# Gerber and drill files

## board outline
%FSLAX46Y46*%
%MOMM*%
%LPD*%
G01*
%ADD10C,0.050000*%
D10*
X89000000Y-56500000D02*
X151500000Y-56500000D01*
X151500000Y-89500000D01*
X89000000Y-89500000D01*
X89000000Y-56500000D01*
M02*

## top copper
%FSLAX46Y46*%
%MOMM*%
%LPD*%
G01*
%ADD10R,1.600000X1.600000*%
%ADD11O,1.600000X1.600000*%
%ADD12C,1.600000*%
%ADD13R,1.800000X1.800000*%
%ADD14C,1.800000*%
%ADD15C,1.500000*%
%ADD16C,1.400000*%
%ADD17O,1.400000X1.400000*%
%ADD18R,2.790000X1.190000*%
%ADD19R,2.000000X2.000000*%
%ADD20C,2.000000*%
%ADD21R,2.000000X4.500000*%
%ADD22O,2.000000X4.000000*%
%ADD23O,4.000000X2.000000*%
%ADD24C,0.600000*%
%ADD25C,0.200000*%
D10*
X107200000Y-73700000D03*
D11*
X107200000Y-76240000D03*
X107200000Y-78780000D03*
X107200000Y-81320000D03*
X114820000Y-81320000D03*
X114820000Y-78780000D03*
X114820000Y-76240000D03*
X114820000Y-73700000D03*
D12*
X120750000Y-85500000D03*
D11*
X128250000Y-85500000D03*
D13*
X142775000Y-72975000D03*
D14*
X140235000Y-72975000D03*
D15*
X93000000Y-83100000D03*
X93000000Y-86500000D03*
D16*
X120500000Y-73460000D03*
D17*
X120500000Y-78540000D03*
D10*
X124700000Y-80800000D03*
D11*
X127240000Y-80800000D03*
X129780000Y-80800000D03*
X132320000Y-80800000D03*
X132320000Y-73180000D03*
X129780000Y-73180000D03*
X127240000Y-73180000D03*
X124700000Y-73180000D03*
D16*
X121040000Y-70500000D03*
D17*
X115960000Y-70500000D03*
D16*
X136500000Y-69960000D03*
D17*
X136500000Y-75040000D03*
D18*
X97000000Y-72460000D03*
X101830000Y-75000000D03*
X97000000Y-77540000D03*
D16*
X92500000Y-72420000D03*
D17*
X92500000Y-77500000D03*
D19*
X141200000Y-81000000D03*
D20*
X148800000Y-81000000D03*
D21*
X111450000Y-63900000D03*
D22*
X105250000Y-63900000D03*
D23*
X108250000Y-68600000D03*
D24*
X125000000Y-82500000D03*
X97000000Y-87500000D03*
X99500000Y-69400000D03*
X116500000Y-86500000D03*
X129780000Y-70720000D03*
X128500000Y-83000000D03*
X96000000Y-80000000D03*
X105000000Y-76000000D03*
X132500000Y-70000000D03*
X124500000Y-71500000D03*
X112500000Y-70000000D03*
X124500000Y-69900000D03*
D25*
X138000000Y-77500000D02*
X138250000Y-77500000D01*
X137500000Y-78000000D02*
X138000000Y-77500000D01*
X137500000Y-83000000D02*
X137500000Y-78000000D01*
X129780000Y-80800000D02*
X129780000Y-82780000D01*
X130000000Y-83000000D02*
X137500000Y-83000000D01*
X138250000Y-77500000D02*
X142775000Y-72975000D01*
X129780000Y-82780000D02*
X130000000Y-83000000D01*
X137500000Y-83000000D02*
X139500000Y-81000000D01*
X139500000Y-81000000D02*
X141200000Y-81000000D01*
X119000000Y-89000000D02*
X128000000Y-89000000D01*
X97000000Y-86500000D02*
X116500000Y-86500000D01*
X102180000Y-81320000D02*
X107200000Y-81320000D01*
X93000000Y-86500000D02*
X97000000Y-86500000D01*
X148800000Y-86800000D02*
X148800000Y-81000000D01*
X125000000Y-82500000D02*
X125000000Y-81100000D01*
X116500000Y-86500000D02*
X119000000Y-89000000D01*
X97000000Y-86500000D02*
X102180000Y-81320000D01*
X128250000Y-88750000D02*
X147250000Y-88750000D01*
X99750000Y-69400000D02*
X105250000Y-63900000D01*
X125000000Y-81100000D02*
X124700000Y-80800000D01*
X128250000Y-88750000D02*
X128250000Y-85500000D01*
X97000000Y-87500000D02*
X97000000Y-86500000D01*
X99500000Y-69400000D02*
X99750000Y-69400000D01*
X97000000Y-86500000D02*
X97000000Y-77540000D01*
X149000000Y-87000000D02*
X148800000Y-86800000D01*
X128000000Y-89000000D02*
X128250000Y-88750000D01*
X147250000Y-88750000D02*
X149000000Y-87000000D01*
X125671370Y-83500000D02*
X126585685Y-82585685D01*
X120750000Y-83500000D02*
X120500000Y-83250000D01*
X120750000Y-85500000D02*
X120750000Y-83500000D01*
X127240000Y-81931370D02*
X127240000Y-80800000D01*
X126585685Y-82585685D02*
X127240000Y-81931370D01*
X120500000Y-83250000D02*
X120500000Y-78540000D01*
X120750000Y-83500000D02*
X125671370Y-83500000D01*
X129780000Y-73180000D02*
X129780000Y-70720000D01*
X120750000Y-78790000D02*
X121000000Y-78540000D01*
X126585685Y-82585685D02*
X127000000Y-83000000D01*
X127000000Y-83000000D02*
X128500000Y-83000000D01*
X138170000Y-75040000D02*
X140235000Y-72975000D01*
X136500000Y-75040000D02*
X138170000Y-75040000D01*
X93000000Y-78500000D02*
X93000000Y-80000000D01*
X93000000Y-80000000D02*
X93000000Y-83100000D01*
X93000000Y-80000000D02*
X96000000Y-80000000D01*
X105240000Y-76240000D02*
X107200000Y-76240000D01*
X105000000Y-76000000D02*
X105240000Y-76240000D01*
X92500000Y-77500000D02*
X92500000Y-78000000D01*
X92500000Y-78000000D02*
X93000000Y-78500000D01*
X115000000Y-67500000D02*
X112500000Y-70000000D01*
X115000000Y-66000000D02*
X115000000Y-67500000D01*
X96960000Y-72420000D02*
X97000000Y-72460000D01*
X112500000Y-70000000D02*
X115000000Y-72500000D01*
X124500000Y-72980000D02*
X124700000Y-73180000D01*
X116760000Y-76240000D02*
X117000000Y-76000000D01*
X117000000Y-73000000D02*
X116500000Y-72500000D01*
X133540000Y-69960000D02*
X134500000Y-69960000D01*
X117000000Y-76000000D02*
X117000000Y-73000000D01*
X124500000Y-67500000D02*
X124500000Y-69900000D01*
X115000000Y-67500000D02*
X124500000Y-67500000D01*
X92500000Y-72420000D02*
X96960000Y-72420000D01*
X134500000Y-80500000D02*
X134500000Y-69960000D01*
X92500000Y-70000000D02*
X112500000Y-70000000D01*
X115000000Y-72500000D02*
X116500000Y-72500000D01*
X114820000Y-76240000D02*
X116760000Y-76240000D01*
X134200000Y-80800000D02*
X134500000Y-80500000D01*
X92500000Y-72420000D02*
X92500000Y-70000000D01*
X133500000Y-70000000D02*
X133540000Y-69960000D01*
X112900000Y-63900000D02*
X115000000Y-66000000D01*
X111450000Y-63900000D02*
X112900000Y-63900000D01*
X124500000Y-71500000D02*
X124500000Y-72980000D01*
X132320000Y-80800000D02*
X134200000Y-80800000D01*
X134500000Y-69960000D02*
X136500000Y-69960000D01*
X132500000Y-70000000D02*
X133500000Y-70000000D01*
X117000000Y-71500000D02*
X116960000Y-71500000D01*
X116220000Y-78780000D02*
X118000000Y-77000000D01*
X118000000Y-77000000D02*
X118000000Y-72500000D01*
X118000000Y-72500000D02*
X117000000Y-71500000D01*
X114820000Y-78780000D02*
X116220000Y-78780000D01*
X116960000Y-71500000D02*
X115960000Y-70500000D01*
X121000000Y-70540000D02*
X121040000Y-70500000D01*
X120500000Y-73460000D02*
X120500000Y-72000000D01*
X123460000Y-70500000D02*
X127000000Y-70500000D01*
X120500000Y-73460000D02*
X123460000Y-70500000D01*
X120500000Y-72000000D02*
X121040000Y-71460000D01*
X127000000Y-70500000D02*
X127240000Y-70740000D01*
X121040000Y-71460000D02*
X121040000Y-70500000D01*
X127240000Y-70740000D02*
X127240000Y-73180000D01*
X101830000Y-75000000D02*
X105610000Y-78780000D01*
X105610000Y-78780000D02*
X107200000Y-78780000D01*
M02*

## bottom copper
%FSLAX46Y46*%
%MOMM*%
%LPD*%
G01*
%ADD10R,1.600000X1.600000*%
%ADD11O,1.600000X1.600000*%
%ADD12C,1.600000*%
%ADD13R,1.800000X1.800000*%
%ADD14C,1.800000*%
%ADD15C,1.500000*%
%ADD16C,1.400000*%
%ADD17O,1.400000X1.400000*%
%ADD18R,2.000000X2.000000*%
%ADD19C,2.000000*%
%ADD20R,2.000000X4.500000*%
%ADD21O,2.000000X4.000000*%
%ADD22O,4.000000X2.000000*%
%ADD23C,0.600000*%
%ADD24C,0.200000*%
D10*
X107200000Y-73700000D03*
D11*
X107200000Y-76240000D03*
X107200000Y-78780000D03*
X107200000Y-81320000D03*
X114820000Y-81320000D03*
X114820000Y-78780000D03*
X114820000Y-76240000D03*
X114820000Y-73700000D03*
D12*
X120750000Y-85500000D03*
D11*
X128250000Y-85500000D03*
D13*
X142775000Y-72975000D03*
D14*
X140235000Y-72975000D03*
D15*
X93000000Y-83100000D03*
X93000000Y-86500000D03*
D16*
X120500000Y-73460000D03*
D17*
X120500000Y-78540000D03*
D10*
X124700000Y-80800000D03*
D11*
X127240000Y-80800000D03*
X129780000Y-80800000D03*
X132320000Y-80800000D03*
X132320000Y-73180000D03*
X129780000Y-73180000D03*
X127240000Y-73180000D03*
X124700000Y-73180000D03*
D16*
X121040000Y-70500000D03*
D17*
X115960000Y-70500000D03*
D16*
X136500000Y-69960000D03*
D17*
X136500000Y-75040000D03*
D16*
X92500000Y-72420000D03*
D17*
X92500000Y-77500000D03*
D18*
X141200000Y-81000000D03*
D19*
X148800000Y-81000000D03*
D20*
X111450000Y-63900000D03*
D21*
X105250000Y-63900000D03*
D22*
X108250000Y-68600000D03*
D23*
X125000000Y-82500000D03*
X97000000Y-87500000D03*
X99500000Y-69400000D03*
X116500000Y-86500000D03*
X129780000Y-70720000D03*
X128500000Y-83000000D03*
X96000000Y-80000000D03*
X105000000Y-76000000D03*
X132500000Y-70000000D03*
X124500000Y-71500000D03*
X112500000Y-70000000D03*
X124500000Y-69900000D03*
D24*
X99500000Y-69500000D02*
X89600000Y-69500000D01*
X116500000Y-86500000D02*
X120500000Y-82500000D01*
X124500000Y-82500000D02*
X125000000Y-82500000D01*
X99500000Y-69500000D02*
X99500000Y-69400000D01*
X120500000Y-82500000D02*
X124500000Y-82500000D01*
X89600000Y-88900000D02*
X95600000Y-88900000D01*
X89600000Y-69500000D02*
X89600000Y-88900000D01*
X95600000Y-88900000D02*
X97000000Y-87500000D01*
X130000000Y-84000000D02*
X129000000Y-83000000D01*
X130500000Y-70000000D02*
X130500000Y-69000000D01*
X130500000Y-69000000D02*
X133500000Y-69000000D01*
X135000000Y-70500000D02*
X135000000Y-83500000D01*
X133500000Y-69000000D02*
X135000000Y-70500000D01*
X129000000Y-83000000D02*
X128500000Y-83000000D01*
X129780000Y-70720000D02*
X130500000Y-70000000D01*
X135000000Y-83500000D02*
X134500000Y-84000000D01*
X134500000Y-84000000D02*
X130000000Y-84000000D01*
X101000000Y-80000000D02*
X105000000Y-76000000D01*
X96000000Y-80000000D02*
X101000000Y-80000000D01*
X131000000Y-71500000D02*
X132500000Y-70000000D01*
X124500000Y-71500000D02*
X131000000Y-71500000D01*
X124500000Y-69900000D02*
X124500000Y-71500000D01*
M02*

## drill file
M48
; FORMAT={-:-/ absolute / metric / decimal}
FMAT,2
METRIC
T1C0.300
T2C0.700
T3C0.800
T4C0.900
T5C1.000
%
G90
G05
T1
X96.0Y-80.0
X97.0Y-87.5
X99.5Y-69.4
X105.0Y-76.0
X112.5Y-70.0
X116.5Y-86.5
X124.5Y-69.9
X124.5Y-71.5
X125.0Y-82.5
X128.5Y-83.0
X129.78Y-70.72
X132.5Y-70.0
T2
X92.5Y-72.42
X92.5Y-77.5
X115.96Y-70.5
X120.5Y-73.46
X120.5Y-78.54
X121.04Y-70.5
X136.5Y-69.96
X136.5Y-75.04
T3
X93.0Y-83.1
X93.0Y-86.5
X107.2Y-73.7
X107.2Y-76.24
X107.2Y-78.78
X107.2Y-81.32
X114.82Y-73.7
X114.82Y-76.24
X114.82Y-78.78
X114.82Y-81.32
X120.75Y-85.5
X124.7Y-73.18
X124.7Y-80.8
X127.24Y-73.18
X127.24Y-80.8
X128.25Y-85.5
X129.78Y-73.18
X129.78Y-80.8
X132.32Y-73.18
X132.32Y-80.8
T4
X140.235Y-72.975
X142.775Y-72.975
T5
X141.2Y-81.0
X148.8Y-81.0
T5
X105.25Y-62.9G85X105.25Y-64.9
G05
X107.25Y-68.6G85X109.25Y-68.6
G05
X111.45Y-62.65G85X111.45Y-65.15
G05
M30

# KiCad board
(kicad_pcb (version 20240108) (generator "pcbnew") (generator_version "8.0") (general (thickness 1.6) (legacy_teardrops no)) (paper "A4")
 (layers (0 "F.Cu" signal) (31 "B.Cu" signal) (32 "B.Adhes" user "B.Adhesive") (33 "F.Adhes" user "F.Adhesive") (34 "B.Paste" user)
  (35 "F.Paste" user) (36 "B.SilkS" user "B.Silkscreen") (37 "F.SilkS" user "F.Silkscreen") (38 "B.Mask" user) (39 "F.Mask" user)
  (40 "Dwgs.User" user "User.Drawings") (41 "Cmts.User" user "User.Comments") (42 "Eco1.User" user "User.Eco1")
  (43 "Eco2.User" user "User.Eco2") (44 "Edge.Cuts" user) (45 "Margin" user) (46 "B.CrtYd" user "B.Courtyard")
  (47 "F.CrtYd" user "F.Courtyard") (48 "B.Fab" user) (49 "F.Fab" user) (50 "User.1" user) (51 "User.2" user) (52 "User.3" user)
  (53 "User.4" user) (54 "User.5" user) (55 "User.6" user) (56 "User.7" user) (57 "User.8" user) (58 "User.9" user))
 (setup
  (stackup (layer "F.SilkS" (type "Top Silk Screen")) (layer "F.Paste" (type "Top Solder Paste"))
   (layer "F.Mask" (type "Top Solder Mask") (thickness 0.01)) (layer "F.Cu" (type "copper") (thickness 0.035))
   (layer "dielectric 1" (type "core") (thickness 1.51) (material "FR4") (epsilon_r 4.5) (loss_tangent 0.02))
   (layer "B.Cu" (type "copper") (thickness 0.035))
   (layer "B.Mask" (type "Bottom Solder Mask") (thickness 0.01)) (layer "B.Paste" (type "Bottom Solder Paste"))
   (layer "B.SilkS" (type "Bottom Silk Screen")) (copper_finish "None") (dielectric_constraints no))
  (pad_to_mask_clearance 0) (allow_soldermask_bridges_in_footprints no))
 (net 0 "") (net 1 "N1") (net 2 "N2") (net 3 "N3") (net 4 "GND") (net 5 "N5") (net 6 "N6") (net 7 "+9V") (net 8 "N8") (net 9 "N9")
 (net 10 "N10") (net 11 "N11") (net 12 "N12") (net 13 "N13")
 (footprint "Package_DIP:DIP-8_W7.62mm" (layer "F.Cu") (at 107.2 73.7)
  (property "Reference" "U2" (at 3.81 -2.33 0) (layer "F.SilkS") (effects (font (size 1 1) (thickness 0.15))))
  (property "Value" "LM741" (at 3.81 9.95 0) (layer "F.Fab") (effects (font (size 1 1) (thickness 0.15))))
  (pad "1" thru_hole rect (at 0 0) (size 1.6 1.6) (drill 0.8) (layers "*.Cu" "*.Mask") (remove_unused_layers no) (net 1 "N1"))
  (pad "2" thru_hole oval (at 0 2.54) (size 1.6 1.6) (drill 0.8) (layers "*.Cu" "*.Mask") (remove_unused_layers no) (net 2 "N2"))
  (pad "3" thru_hole oval (at 0 5.08) (size 1.6 1.6) (drill 0.8) (layers "*.Cu" "*.Mask") (remove_unused_layers no) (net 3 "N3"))
  (pad "4" thru_hole oval (at 0 7.62) (size 1.6 1.6) (drill 0.8) (layers "*.Cu" "*.Mask") (remove_unused_layers no) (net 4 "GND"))
  (pad "5" thru_hole oval (at 7.62 7.62) (size 1.6 1.6) (drill 0.8) (layers "*.Cu" "*.Mask") (remove_unused_layers no) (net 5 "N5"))
  (pad "6" thru_hole oval (at 7.62 5.08) (size 1.6 1.6) (drill 0.8) (layers "*.Cu" "*.Mask") (remove_unused_layers no) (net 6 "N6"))
  (pad "7" thru_hole oval (at 7.62 2.54) (size 1.6 1.6) (drill 0.8) (layers "*.Cu" "*.Mask") (remove_unused_layers no) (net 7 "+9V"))
  (pad "8" thru_hole oval (at 7.62 0) (size 1.6 1.6) (drill 0.8) (layers "*.Cu" "*.Mask") (remove_unused_layers no) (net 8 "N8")))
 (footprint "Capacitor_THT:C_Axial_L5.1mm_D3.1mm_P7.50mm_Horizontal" (layer "F.Cu") (at 120.75 85.5)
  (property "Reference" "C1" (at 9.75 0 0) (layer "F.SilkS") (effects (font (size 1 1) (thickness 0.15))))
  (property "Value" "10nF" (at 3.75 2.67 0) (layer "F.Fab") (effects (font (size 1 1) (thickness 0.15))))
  (pad "1" thru_hole circle (at 0 0) (size 1.6 1.6) (drill 0.8) (layers "*.Cu" "*.Mask") (remove_unused_layers no) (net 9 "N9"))
  (pad "2" thru_hole oval (at 7.5 0) (size 1.6 1.6) (drill 0.8) (layers "*.Cu" "*.Mask") (remove_unused_layers no) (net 4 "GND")))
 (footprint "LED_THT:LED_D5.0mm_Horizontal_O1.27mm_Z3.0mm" (layer "F.Cu") (at 142.775 72.975 180)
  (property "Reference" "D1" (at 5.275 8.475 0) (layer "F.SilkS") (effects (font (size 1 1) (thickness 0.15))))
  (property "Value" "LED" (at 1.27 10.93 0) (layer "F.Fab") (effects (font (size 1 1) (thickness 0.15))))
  (pad "1" thru_hole rect (at 0 0 180) (size 1.8 1.8) (drill 0.9) (layers "*.Cu" "*.Mask") (remove_unused_layers no) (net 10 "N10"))
  (pad "2" thru_hole circle (at 2.54 0 180) (size 1.8 1.8) (drill 0.9) (layers "*.Cu" "*.Mask") (remove_unused_layers no) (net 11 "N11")))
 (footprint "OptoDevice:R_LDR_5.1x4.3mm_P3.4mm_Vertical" (layer "F.Cu") (at 93 83.1 -90)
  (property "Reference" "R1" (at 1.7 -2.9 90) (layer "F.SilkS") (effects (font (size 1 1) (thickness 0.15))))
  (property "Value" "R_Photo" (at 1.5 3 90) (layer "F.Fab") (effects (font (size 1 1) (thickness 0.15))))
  (pad "1" thru_hole circle (at 0 0 270) (size 1.5 1.5) (drill 0.8) (layers "*.Cu" "*.Mask") (remove_unused_layers no) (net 2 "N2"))
  (pad "2" thru_hole circle (at 3.4 0 270) (size 1.5 1.5) (drill 0.8) (layers "*.Cu" "*.Mask") (remove_unused_layers no) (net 4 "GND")))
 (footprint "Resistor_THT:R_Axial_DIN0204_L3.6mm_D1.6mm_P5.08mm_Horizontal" (layer "F.Cu") (at 120.5 73.46 -90)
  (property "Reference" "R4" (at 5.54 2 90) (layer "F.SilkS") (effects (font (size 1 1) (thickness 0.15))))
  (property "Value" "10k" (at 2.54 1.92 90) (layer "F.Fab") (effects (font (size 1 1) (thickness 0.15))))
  (pad "1" thru_hole circle (at 0 0 270) (size 1.4 1.4) (drill 0.7) (layers "*.Cu" "*.Mask") (remove_unused_layers no) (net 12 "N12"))
  (pad "2" thru_hole oval (at 5.08 0 270) (size 1.4 1.4) (drill 0.7) (layers "*.Cu" "*.Mask") (remove_unused_layers no) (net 9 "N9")))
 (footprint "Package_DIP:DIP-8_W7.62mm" (layer "F.Cu") (at 124.7 80.8 90)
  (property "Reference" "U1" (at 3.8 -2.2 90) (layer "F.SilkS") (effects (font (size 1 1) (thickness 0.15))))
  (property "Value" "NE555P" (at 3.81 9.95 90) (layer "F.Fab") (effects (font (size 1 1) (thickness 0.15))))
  (pad "1" thru_hole rect (at 0 0 90) (size 1.6 1.6) (drill 0.8) (layers "*.Cu" "*.Mask") (remove_unused_layers no) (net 4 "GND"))
  (pad "2" thru_hole oval (at 0 2.54 90) (size 1.6 1.6) (drill 0.8) (layers "*.Cu" "*.Mask") (remove_unused_layers no) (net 9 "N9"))
  (pad "3" thru_hole oval (at 0 5.08 90) (size 1.6 1.6) (drill 0.8) (layers "*.Cu" "*.Mask") (remove_unused_layers no) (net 10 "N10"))
  (pad "4" thru_hole oval (at 0 7.62 90) (size 1.6 1.6) (drill 0.8) (layers "*.Cu" "*.Mask") (remove_unused_layers no) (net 7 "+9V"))
  (pad "5" thru_hole oval (at 7.62 7.62 90) (size 1.6 1.6) (drill 0.8) (layers "*.Cu" "*.Mask") (remove_unused_layers no) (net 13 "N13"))
  (pad "6" thru_hole oval (at 7.62 5.08 90) (size 1.6 1.6) (drill 0.8) (layers "*.Cu" "*.Mask") (remove_unused_layers no) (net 9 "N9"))
  (pad "7" thru_hole oval (at 7.62 2.54 90) (size 1.6 1.6) (drill 0.8) (layers "*.Cu" "*.Mask") (remove_unused_layers no) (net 12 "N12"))
  (pad "8" thru_hole oval (at 7.62 0 90) (size 1.6 1.6) (drill 0.8) (layers "*.Cu" "*.Mask") (remove_unused_layers no) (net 7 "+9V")))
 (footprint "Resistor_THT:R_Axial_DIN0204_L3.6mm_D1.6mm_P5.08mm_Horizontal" (layer "F.Cu") (at 121.04 70.5 180)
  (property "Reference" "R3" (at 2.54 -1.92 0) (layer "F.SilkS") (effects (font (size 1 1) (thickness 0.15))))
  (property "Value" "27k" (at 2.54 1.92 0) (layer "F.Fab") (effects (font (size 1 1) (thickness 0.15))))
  (pad "1" thru_hole circle (at 0 0 180) (size 1.4 1.4) (drill 0.7) (layers "*.Cu" "*.Mask") (remove_unused_layers no) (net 12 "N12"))
  (pad "2" thru_hole oval (at 5.08 0 180) (size 1.4 1.4) (drill 0.7) (layers "*.Cu" "*.Mask") (remove_unused_layers no) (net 6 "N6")))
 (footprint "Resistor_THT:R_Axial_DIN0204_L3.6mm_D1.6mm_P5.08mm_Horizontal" (layer "F.Cu") (at 136.5 69.96 -90)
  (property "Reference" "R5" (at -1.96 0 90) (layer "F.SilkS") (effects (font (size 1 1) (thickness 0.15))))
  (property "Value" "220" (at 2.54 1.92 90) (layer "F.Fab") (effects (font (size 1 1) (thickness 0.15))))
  (pad "1" thru_hole circle (at 0 0 270) (size 1.4 1.4) (drill 0.7) (layers "*.Cu" "*.Mask") (remove_unused_layers no) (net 7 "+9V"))
  (pad "2" thru_hole oval (at 5.08 0 270) (size 1.4 1.4) (drill 0.7) (layers "*.Cu" "*.Mask") (remove_unused_layers no) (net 11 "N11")))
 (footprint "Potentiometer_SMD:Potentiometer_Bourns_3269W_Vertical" (layer "F.Cu") (at 99.415 75 90)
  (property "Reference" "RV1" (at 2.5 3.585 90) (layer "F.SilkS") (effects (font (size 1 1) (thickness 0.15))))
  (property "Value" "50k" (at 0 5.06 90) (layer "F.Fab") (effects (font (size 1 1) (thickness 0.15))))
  (pad "1" smd rect (at 2.54 -2.415 90) (size 1.19 2.79) (layers "F.Cu" "F.Paste" "F.Mask") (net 7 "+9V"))
  (pad "2" smd rect (at 0 2.415 90) (size 1.19 2.79) (layers "F.Cu" "F.Paste" "F.Mask") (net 3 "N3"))
  (pad "3" smd rect (at -2.54 -2.415 90) (size 1.19 2.79) (layers "F.Cu" "F.Paste" "F.Mask") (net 4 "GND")))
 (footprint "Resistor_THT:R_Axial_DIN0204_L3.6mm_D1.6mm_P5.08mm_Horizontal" (layer "F.Cu") (at 92.5 72.42 -90)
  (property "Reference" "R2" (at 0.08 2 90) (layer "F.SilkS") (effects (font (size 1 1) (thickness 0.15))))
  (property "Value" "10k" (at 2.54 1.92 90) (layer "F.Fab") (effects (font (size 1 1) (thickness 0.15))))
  (pad "1" thru_hole circle (at 0 0 270) (size 1.4 1.4) (drill 0.7) (layers "*.Cu" "*.Mask") (remove_unused_layers no) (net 7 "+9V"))
  (pad "2" thru_hole oval (at 5.08 0 270) (size 1.4 1.4) (drill 0.7) (layers "*.Cu" "*.Mask") (remove_unused_layers no) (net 2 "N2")))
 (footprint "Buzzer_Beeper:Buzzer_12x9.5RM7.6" (layer "F.Cu") (at 141.2 81)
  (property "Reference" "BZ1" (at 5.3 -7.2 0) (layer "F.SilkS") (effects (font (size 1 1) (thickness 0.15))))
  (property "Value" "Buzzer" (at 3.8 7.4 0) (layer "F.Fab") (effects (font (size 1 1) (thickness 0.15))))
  (pad "1" thru_hole rect (at 0 0) (size 2 2) (drill 1) (layers "*.Cu" "*.Mask") (remove_unused_layers no) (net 10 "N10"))
  (pad "2" thru_hole circle (at 7.6 0) (size 2 2) (drill 1) (layers "*.Cu" "*.Mask") (remove_unused_layers no) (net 4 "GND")))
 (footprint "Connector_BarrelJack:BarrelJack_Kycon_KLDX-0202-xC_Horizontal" (layer "F.Cu") (at 111.45 63.9)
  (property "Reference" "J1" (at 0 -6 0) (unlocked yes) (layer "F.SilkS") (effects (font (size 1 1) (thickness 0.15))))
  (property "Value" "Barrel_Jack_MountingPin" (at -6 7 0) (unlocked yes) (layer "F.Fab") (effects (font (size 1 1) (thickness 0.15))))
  (pad "1" thru_hole rect (at 0 0) (size 2 4.5) (drill oval 1 3.5) (layers "*.Cu" "*.Mask") (remove_unused_layers no) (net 7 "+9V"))
  (pad "2" thru_hole oval (at -6.2 0) (size 2 4) (drill oval 1 3) (layers "*.Cu" "*.Mask") (remove_unused_layers no) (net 4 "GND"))
  (pad "3" thru_hole oval (at -3.2 4.7 90) (size 2 4) (drill oval 1 3) (layers "*.Cu" "*.Mask") (remove_unused_layers no)))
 (gr_rect (start 89 56.5) (end 151.5 89.5) (stroke (width 0.05) (type default)) (fill none) (layer "Edge.Cuts"))
 (segment (start 138 77.5) (end 138.25 77.5) (width 0.2) (layer "F.Cu") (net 10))
 (segment (start 137.5 78) (end 138 77.5) (width 0.2) (layer "F.Cu") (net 10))
 (segment (start 137.5 83) (end 137.5 78) (width 0.2) (layer "F.Cu") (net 10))
 (segment (start 129.78 80.8) (end 129.78 82.78) (width 0.2) (layer "F.Cu") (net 10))
 (segment (start 130 83) (end 137.5 83) (width 0.2) (layer "F.Cu") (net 10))
 (segment (start 138.25 77.5) (end 142.775 72.975) (width 0.2) (layer "F.Cu") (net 10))
 (segment (start 129.78 82.78) (end 130 83) (width 0.2) (layer "F.Cu") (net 10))
 (segment (start 137.5 83) (end 139.5 81) (width 0.2) (layer "F.Cu") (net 10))
 (segment (start 139.5 81) (end 141.2 81) (width 0.2) (layer "F.Cu") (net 10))
 (segment (start 119 89) (end 128 89) (width 0.2) (layer "F.Cu") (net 4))
 (segment (start 97 86.5) (end 116.5 86.5) (width 0.2) (layer "F.Cu") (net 4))
 (segment (start 102.18 81.32) (end 107.2 81.32) (width 0.2) (layer "F.Cu") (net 4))
 (segment (start 93 86.5) (end 97 86.5) (width 0.2) (layer "F.Cu") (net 4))
 (segment (start 148.8 86.8) (end 148.8 81) (width 0.2) (layer "F.Cu") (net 4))
 (segment (start 125 82.5) (end 125 81.1) (width 0.2) (layer "F.Cu") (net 4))
 (segment (start 116.5 86.5) (end 119 89) (width 0.2) (layer "F.Cu") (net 4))
 (segment (start 97 86.5) (end 102.18 81.32) (width 0.2) (layer "F.Cu") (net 4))
 (segment (start 128.25 88.75) (end 147.25 88.75) (width 0.2) (layer "F.Cu") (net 4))
 (segment (start 99.75 69.4) (end 105.25 63.9) (width 0.2) (layer "F.Cu") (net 4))
 (segment (start 125 81.1) (end 124.7 80.8) (width 0.2) (layer "F.Cu") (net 4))
 (segment (start 128.25 88.75) (end 128.25 85.5) (width 0.2) (layer "F.Cu") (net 4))
 (segment (start 97 87.5) (end 97 86.5) (width 0.2) (layer "F.Cu") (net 4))
 (segment (start 99.5 69.4) (end 99.75 69.4) (width 0.2) (layer "F.Cu") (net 4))
 (segment (start 97 86.5) (end 97 77.54) (width 0.2) (layer "F.Cu") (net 4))
 (segment (start 149 87) (end 148.8 86.8) (width 0.2) (layer "F.Cu") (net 4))
 (segment (start 128 89) (end 128.25 88.75) (width 0.2) (layer "F.Cu") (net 4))
 (segment (start 147.25 88.75) (end 149 87) (width 0.2) (layer "F.Cu") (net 4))
 (via (at 125 82.5) (size 0.6) (drill 0.3) (layers "F.Cu" "B.Cu") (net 4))
 (via (at 97 87.5) (size 0.6) (drill 0.3) (layers "F.Cu" "B.Cu") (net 4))
 (via (at 99.5 69.4) (size 0.6) (drill 0.3) (layers "F.Cu" "B.Cu") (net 4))
 (via (at 116.5 86.5) (size 0.6) (drill 0.3) (layers "F.Cu" "B.Cu") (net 4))
 (segment (start 99.5 69.5) (end 89.6 69.5) (width 0.2) (layer "B.Cu") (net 4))
 (segment (start 116.5 86.5) (end 120.5 82.5) (width 0.2) (layer "B.Cu") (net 4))
 (segment (start 124.5 82.5) (end 125 82.5) (width 0.2) (layer "B.Cu") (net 4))
 (segment (start 99.5 69.5) (end 99.5 69.4) (width 0.2) (layer "B.Cu") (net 4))
 (segment (start 120.5 82.5) (end 124.5 82.5) (width 0.2) (layer "B.Cu") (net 4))
 (segment (start 89.6 88.9) (end 95.6 88.9) (width 0.2) (layer "B.Cu") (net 4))
 (segment (start 89.6 69.5) (end 89.6 88.9) (width 0.2) (layer "B.Cu") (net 4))
 (segment (start 95.6 88.9) (end 97 87.5) (width 0.2) (layer "B.Cu") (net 4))
 (segment (start 125.67137 83.5) (end 126.585685 82.585685) (width 0.2) (layer "F.Cu") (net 9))
 (segment (start 120.75 83.5) (end 120.5 83.25) (width 0.2) (layer "F.Cu") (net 9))
 (segment (start 120.75 85.5) (end 120.75 83.5) (width 0.2) (layer "F.Cu") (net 9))
 (segment (start 127.24 81.93137) (end 127.24 80.8) (width 0.2) (layer "F.Cu") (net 9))
 (segment (start 126.585685 82.585685) (end 127.24 81.93137) (width 0.2) (layer "F.Cu") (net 9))
 (segment (start 120.5 83.25) (end 120.5 78.54) (width 0.2) (layer "F.Cu") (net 9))
 (segment (start 120.75 83.5) (end 125.67137 83.5) (width 0.2) (layer "F.Cu") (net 9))
 (segment (start 129.78 73.18) (end 129.78 70.72) (width 0.2) (layer "F.Cu") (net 9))
 (segment (start 120.75 78.79) (end 121 78.54) (width 0.2) (layer "F.Cu") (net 9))
 (segment (start 126.585685 82.585685) (end 127 83) (width 0.2) (layer "F.Cu") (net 9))
 (segment (start 127 83) (end 128.5 83) (width 0.2) (layer "F.Cu") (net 9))
 (via (at 129.78 70.72) (size 0.6) (drill 0.3) (layers "F.Cu" "B.Cu") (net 9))
 (via (at 128.5 83) (size 0.6) (drill 0.3) (layers "F.Cu" "B.Cu") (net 9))
 (segment (start 130 84) (end 129 83) (width 0.2) (layer "B.Cu") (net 9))
 (segment (start 130.5 70) (end 130.5 69) (width 0.2) (layer "B.Cu") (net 9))
 (segment (start 130.5 69) (end 133.5 69) (width 0.2) (layer "B.Cu") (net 9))
 (segment (start 135 70.5) (end 135 83.5) (width 0.2) (layer "B.Cu") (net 9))
 (segment (start 133.5 69) (end 135 70.5) (width 0.2) (layer "B.Cu") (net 9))
 (segment (start 129 83) (end 128.5 83) (width 0.2) (layer "B.Cu") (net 9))
 (segment (start 129.78 70.72) (end 130.5 70) (width 0.2) (layer "B.Cu") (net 9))
 (segment (start 135 83.5) (end 134.5 84) (width 0.2) (layer "B.Cu") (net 9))
 (segment (start 134.5 84) (end 130 84) (width 0.2) (layer "B.Cu") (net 9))
 (segment (start 138.17 75.04) (end 140.235 72.975) (width 0.2) (layer "F.Cu") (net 11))
 (segment (start 136.5 75.04) (end 138.17 75.04) (width 0.2) (layer "F.Cu") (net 11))
 (segment (start 93 78.5) (end 93 80) (width 0.2) (layer "F.Cu") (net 2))
 (segment (start 93 80) (end 93 83.1) (width 0.2) (layer "F.Cu") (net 2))
 (segment (start 93 80) (end 96 80) (width 0.2) (layer "F.Cu") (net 2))
 (segment (start 105.24 76.24) (end 107.2 76.24) (width 0.2) (layer "F.Cu") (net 2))
 (segment (start 105 76) (end 105.24 76.24) (width 0.2) (layer "F.Cu") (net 2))
 (segment (start 92.5 77.5) (end 92.5 78) (width 0.2) (layer "F.Cu") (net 2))
 (segment (start 92.5 78) (end 93 78.5) (width 0.2) (layer "F.Cu") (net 2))
 (via (at 96 80) (size 0.6) (drill 0.3) (layers "F.Cu" "B.Cu") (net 2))
 (via (at 105 76) (size 0.6) (drill 0.3) (layers "F.Cu" "B.Cu") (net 2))
 (segment (start 101 80) (end 105 76) (width 0.2) (layer "B.Cu") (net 2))
 (segment (start 96 80) (end 101 80) (width 0.2) (layer "B.Cu") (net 2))
 (segment (start 115 67.5) (end 112.5 70) (width 0.2) (layer "F.Cu") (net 7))
 (segment (start 115 66) (end 115 67.5) (width 0.2) (layer "F.Cu") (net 7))
 (segment (start 96.96 72.42) (end 97 72.46) (width 0.2) (layer "F.Cu") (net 7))
 (segment (start 112.5 70) (end 115 72.5) (width 0.2) (layer "F.Cu") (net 7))
 (segment (start 124.5 72.98) (end 124.7 73.18) (width 0.2) (layer "F.Cu") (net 7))
 (segment (start 116.76 76.24) (end 117 76) (width 0.2) (layer "F.Cu") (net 7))
 (segment (start 117 73) (end 116.5 72.5) (width 0.2) (layer "F.Cu") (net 7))
 (segment (start 133.54 69.96) (end 134.5 69.96) (width 0.2) (layer "F.Cu") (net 7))
 (segment (start 117 76) (end 117 73) (width 0.2) (layer "F.Cu") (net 7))
 (segment (start 124.5 67.5) (end 124.5 69.9) (width 0.2) (layer "F.Cu") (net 7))
 (segment (start 115 67.5) (end 124.5 67.5) (width 0.2) (layer "F.Cu") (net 7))
 (segment (start 92.5 72.42) (end 96.96 72.42) (width 0.2) (layer "F.Cu") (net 7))
 (segment (start 134.5 80.5) (end 134.5 69.96) (width 0.2) (layer "F.Cu") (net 7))
 (segment (start 92.5 70) (end 112.5 70) (width 0.2) (layer "F.Cu") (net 7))
 (segment (start 115 72.5) (end 116.5 72.5) (width 0.2) (layer "F.Cu") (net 7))
 (segment (start 114.82 76.24) (end 116.76 76.24) (width 0.2) (layer "F.Cu") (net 7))
 (segment (start 134.2 80.8) (end 134.5 80.5) (width 0.2) (layer "F.Cu") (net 7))
 (segment (start 92.5 72.42) (end 92.5 70) (width 0.2) (layer "F.Cu") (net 7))
 (segment (start 133.5 70) (end 133.54 69.96) (width 0.2) (layer "F.Cu") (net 7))
 (segment (start 112.9 63.9) (end 115 66) (width 0.2) (layer "F.Cu") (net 7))
 (segment (start 111.45 63.9) (end 112.9 63.9) (width 0.2) (layer "F.Cu") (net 7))
 (segment (start 124.5 71.5) (end 124.5 72.98) (width 0.2) (layer "F.Cu") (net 7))
 (segment (start 132.32 80.8) (end 134.2 80.8) (width 0.2) (layer "F.Cu") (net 7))
 (segment (start 134.5 69.96) (end 136.5 69.96) (width 0.2) (layer "F.Cu") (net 7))
 (segment (start 132.5 70) (end 133.5 70) (width 0.2) (layer "F.Cu") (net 7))
 (via (at 132.5 70) (size 0.6) (drill 0.3) (layers "F.Cu" "B.Cu") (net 7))
 (via (at 124.5 71.5) (size 0.6) (drill 0.3) (layers "F.Cu" "B.Cu") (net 7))
 (via (at 112.5 70) (size 0.6) (drill 0.3) (layers "F.Cu" "B.Cu") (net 7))
 (via (at 124.5 69.9) (size 0.6) (drill 0.3) (layers "F.Cu" "B.Cu") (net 7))
 (segment (start 131 71.5) (end 132.5 70) (width 0.2) (layer "B.Cu") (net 7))
 (segment (start 124.5 71.5) (end 131 71.5) (width 0.2) (layer "B.Cu") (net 7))
 (segment (start 124.5 69.9) (end 124.5 71.5) (width 0.2) (layer "B.Cu") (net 7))
 (segment (start 117 71.5) (end 116.96 71.5) (width 0.2) (layer "F.Cu") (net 6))
 (segment (start 116.22 78.78) (end 118 77) (width 0.2) (layer "F.Cu") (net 6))
 (segment (start 118 77) (end 118 72.5) (width 0.2) (layer "F.Cu") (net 6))
 (segment (start 118 72.5) (end 117 71.5) (width 0.2) (layer "F.Cu") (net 6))
 (segment (start 114.82 78.78) (end 116.22 78.78) (width 0.2) (layer "F.Cu") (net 6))
 (segment (start 116.96 71.5) (end 115.96 70.5) (width 0.2) (layer "F.Cu") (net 6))
 (segment (start 121 70.54) (end 121.04 70.5) (width 0.2) (layer "F.Cu") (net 12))
 (segment (start 120.5 73.46) (end 120.5 72) (width 0.2) (layer "F.Cu") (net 12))
 (segment (start 123.46 70.5) (end 127 70.5) (width 0.2) (layer "F.Cu") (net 12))
 (segment (start 120.5 73.46) (end 123.46 70.5) (width 0.2) (layer "F.Cu") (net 12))
 (segment (start 120.5 72) (end 121.04 71.46) (width 0.2) (layer "F.Cu") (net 12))
 (segment (start 127 70.5) (end 127.24 70.74) (width 0.2) (layer "F.Cu") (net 12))
 (segment (start 121.04 71.46) (end 121.04 70.5) (width 0.2) (layer "F.Cu") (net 12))
 (segment (start 127.24 70.74) (end 127.24 73.18) (width 0.2) (layer "F.Cu") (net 12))
 (segment (start 101.83 75) (end 105.61 78.78) (width 0.2) (layer "F.Cu") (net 3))
 (segment (start 105.61 78.78) (end 107.2 78.78) (width 0.2) (layer "F.Cu") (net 3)))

